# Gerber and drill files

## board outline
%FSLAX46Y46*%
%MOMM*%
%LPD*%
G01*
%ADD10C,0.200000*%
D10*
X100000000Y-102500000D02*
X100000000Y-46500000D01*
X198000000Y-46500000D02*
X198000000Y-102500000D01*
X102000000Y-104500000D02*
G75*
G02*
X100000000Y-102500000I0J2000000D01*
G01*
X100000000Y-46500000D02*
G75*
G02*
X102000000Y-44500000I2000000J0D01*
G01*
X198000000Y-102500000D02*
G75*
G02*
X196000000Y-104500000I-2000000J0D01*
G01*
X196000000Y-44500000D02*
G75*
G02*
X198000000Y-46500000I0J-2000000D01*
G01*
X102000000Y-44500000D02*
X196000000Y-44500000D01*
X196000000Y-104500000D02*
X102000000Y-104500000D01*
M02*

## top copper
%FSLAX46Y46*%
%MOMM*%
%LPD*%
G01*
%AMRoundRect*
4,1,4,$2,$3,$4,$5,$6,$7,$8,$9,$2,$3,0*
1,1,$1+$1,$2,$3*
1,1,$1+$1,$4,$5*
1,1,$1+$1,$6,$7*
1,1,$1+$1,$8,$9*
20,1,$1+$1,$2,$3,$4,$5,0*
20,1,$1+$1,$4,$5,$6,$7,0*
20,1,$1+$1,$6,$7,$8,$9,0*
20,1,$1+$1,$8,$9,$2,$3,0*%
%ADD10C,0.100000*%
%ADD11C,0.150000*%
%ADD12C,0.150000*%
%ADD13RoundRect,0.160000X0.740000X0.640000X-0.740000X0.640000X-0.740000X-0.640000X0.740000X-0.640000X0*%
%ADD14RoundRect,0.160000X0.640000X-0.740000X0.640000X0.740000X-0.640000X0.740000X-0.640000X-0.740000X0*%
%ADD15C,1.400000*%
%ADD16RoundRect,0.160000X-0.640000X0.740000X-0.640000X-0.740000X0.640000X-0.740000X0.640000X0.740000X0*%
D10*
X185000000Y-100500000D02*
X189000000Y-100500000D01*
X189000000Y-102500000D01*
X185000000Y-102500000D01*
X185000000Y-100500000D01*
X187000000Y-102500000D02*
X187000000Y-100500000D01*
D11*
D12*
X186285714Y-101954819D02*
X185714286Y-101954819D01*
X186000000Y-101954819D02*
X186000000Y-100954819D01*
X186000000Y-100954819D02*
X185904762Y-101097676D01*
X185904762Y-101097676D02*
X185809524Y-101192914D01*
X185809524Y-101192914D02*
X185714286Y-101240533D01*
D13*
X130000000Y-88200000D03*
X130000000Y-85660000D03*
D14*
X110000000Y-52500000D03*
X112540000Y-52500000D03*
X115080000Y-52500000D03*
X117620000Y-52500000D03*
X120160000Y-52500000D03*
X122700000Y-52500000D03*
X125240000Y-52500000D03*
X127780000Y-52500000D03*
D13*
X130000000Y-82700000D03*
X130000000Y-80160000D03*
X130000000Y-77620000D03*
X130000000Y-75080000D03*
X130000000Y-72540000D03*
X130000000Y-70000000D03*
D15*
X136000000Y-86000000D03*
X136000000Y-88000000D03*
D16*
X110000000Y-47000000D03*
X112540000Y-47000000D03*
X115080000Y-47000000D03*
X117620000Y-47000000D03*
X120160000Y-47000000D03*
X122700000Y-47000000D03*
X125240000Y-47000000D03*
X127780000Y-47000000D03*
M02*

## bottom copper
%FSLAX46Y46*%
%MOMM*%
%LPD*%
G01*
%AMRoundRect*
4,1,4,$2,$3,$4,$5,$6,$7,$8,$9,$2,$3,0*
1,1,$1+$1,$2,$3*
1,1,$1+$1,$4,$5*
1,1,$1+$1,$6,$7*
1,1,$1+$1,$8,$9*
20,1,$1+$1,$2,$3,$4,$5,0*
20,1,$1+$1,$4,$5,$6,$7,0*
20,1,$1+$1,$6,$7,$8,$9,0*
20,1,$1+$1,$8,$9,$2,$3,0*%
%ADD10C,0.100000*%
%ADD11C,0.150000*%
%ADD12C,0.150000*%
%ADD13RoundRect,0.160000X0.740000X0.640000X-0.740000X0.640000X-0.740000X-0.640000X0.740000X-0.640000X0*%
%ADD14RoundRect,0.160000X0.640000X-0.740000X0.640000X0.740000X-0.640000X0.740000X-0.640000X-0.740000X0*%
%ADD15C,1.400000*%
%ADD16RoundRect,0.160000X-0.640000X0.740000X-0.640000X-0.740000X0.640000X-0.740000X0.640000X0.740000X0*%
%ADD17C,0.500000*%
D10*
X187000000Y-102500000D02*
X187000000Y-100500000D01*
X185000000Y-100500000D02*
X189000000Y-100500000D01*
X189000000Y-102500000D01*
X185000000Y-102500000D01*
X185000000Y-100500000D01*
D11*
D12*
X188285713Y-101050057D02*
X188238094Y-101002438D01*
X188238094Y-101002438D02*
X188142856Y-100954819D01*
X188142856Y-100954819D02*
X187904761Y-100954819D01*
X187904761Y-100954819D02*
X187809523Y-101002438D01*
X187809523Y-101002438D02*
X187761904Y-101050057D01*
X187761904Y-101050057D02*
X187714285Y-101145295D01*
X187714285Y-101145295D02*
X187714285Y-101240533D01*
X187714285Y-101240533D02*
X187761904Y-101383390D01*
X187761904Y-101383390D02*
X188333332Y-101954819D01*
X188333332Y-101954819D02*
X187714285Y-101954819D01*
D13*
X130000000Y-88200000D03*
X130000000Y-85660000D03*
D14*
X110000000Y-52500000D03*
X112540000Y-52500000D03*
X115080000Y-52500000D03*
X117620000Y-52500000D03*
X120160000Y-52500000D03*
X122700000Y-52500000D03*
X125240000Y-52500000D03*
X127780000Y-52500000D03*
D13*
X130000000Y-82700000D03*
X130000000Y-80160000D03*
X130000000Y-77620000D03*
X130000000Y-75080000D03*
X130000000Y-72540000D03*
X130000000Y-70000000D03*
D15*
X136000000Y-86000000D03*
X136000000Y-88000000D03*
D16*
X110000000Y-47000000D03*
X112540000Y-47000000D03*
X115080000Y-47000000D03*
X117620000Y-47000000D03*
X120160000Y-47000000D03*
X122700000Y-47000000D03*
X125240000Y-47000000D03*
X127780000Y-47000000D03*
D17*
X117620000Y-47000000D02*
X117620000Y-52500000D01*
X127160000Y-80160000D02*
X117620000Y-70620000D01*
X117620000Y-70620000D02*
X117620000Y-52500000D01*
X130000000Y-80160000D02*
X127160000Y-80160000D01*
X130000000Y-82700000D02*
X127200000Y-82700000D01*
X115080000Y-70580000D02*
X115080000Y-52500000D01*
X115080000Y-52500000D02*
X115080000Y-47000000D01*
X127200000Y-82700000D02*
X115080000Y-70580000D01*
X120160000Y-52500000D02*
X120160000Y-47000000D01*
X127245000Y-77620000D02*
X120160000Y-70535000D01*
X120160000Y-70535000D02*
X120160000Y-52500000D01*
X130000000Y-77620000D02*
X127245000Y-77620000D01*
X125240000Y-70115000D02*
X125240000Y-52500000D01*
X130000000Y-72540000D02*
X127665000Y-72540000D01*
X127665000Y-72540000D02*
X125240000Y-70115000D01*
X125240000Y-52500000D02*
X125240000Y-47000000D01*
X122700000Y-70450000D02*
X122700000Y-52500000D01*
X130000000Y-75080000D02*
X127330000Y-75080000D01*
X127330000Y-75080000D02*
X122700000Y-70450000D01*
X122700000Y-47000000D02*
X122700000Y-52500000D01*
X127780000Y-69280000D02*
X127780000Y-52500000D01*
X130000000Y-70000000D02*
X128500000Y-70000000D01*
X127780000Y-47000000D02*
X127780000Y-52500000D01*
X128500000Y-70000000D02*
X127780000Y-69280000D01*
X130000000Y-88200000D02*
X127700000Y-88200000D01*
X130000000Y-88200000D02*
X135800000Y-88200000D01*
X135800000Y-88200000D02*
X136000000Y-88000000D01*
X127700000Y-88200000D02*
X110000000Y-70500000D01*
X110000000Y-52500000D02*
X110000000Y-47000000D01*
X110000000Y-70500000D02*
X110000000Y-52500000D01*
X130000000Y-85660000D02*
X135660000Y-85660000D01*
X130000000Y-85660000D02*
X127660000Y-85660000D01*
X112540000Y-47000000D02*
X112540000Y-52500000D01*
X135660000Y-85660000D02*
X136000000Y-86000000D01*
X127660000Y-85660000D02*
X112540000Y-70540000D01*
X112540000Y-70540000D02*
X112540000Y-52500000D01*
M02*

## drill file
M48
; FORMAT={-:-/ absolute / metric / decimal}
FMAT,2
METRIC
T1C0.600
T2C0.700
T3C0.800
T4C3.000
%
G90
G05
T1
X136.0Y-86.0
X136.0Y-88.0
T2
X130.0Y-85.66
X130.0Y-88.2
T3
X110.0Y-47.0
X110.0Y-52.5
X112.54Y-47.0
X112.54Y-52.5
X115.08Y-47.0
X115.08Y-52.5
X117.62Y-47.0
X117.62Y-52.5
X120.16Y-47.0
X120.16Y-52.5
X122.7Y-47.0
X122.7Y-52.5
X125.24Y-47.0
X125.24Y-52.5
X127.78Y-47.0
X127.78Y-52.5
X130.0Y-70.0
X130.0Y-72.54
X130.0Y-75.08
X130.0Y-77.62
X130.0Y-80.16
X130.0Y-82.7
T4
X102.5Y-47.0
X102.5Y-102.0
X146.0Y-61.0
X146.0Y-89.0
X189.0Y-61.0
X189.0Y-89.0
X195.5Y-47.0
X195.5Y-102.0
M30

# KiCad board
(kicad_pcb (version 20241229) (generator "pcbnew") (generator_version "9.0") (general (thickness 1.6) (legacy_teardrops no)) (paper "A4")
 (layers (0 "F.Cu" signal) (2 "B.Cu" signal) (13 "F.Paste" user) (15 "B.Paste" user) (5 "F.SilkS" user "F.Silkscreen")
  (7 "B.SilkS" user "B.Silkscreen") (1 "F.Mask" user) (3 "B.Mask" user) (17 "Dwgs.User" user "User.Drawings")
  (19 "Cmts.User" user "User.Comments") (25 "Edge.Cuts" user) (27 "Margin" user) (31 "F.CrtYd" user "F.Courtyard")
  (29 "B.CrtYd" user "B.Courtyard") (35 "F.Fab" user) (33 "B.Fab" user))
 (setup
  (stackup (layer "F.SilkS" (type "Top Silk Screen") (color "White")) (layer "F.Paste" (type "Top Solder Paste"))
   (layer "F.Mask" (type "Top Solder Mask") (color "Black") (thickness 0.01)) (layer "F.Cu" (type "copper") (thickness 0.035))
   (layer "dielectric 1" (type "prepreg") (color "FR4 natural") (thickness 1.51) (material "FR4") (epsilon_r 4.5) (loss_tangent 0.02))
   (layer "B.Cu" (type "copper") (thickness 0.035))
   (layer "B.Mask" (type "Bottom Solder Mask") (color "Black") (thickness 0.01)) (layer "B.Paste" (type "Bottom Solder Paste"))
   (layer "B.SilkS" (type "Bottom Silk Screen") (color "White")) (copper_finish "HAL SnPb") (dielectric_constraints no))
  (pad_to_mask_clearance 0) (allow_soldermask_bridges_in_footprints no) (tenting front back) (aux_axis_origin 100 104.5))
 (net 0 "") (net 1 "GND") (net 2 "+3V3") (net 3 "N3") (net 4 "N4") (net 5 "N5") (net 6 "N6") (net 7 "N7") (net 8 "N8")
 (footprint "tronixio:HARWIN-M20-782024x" (layer "F.Cu") (at 130 88.2 180)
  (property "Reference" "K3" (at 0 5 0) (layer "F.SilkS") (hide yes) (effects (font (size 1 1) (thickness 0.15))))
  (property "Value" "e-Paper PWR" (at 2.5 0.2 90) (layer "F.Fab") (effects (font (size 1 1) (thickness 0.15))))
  (pad "1" thru_hole roundrect (at 0 0 180) (size 1.8 1.6) (drill 0.7) (layers "*.Cu" "*.Mask") (remove_unused_layers no)
   (roundrect_rratio 0.1) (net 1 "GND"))
  (pad "2" thru_hole roundrect (at 0 2.54 180) (size 1.8 1.6) (drill 0.7) (layers "*.Cu" "*.Mask") (remove_unused_layers no)
   (roundrect_rratio 0.1) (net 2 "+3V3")))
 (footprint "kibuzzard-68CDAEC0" (layer "F.Cu") (at 112.54 57 90)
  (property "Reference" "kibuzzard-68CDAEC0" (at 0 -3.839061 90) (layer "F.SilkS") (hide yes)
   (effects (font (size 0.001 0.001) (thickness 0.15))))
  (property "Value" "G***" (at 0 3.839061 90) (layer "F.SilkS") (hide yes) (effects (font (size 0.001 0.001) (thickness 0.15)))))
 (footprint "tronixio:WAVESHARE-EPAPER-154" (layer "F.Cu") (at 167.5 75)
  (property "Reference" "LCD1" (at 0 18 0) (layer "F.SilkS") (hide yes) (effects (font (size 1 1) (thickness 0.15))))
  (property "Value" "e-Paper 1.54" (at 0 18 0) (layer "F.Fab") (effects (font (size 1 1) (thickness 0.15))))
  (pad "" np_thru_hole circle (at -21.5 -14) (size 3 3) (drill 3) (layers "*.Cu" "*.Mask"))
  (pad "" np_thru_hole circle (at -21.5 14) (size 3 3) (drill 3) (layers "*.Cu" "*.Mask"))
  (pad "" np_thru_hole circle (at 21.5 -14) (size 3 3) (drill 3) (layers "*.Cu" "*.Mask"))
  (pad "" np_thru_hole circle (at 21.5 14) (size 3 3) (drill 3) (layers "*.Cu" "*.Mask")))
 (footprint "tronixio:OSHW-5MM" (layer "F.Cu") (at 167.5 67.5)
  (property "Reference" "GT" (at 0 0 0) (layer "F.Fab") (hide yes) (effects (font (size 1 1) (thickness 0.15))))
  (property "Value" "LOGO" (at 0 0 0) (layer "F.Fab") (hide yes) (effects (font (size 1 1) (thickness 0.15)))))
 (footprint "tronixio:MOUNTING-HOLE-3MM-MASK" (layer "F.Cu") (at 195.5 102)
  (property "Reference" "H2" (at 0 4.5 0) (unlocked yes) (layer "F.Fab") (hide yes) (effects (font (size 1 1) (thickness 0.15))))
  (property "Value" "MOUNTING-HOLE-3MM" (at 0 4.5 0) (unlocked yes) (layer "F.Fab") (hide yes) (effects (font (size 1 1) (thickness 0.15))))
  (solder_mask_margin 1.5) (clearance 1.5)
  (pad "" np_thru_hole circle (at 0 0) (size 3 3) (drill 3) (layers "*.Cu" "*.Mask")))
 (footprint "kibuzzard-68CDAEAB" (layer "F.Cu") (at 126 88.5)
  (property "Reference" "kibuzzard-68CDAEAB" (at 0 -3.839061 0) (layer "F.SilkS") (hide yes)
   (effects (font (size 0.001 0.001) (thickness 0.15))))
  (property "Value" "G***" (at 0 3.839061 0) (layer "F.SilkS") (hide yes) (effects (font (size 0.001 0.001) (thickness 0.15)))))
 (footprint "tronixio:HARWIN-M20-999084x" (layer "F.Cu") (at 110 52.5 90)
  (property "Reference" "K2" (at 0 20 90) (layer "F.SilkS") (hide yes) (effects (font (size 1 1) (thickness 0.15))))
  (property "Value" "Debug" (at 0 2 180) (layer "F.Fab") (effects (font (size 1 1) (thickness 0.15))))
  (pad "1" thru_hole roundrect (at 0 0 90) (size 1.8 1.6) (drill 0.8) (layers "*.Cu" "*.Mask") (remove_unused_layers no)
   (roundrect_rratio 0.1) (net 1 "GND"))
  (pad "2" thru_hole roundrect (at 0 2.54 90) (size 1.8 1.6) (drill 0.8) (layers "*.Cu" "*.Mask") (remove_unused_layers no)
   (roundrect_rratio 0.1) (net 2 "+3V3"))
  (pad "3" thru_hole roundrect (at 0 5.08 90) (size 1.8 1.6) (drill 0.8) (layers "*.Cu" "*.Mask") (remove_unused_layers no)
   (roundrect_rratio 0.1) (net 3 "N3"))
  (pad "4" thru_hole roundrect (at 0 7.62 90) (size 1.8 1.6) (drill 0.8) (layers "*.Cu" "*.Mask") (remove_unused_layers no)
   (roundrect_rratio 0.1) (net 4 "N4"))
  (pad "5" thru_hole roundrect (at 0 10.16 90) (size 1.8 1.6) (drill 0.8) (layers "*.Cu" "*.Mask") (remove_unused_layers no)
   (roundrect_rratio 0.1) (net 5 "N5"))
  (pad "6" thru_hole roundrect (at 0 12.7 90) (size 1.8 1.6) (drill 0.8) (layers "*.Cu" "*.Mask") (remove_unused_layers no)
   (roundrect_rratio 0.1) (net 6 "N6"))
  (pad "7" thru_hole roundrect (at 0 15.24 90) (size 1.8 1.6) (drill 0.8) (layers "*.Cu" "*.Mask") (remove_unused_layers no)
   (roundrect_rratio 0.1) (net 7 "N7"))
  (pad "8" thru_hole roundrect (at 0 17.78 90) (size 1.8 1.6) (drill 0.8) (layers "*.Cu" "*.Mask") (remove_unused_layers no)
   (roundrect_rratio 0.1) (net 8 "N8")))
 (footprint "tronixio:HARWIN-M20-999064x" (layer "F.Cu") (at 130 82.7 180)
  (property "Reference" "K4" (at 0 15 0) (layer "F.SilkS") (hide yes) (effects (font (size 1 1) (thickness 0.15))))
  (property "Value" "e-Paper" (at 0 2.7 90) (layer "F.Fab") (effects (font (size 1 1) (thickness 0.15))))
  (pad "1" thru_hole roundrect (at 0 0 180) (size 1.8 1.6) (drill 0.8) (layers "*.Cu" "*.Mask") (remove_unused_layers no)
   (roundrect_rratio 0.1) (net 3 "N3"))
  (pad "2" thru_hole roundrect (at 0 2.54 180) (size 1.8 1.6) (drill 0.8) (layers "*.Cu" "*.Mask") (remove_unused_layers no)
   (roundrect_rratio 0.1) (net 4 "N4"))
  (pad "3" thru_hole roundrect (at 0 5.08 180) (size 1.8 1.6) (drill 0.8) (layers "*.Cu" "*.Mask") (remove_unused_layers no)
   (roundrect_rratio 0.1) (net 5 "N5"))
  (pad "4" thru_hole roundrect (at 0 7.62 180) (size 1.8 1.6) (drill 0.8) (layers "*.Cu" "*.Mask") (remove_unused_layers no)
   (roundrect_rratio 0.1) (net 6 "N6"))
  (pad "5" thru_hole roundrect (at 0 10.16 180) (size 1.8 1.6) (drill 0.8) (layers "*.Cu" "*.Mask") (remove_unused_layers no)
   (roundrect_rratio 0.1) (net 7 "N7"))
  (pad "6" thru_hole roundrect (at 0 12.7 180) (size 1.8 1.6) (drill 0.8) (layers "*.Cu" "*.Mask") (remove_unused_layers no)
   (roundrect_rratio 0.1) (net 8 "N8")))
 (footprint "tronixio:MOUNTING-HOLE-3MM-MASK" (layer "F.Cu") (at 102.5 47)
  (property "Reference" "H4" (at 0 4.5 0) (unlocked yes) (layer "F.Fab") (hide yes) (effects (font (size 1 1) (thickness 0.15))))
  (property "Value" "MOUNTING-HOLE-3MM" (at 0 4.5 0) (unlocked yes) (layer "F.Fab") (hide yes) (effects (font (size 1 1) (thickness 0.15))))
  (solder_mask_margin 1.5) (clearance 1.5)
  (pad "" np_thru_hole circle (at 0 0) (size 3 3) (drill 3) (layers "*.Cu" "*.Mask")))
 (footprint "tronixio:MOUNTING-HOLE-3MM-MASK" (layer "F.Cu") (at 195.5 47)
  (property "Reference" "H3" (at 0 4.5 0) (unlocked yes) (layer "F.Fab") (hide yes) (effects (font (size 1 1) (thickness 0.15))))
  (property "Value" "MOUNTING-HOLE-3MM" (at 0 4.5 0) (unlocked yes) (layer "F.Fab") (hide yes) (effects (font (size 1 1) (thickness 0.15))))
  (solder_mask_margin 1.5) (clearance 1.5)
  (pad "" np_thru_hole circle (at 0 0) (size 3 3) (drill 3) (layers "*.Cu" "*.Mask")))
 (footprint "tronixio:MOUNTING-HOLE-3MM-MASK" (layer "F.Cu") (at 102.5 102)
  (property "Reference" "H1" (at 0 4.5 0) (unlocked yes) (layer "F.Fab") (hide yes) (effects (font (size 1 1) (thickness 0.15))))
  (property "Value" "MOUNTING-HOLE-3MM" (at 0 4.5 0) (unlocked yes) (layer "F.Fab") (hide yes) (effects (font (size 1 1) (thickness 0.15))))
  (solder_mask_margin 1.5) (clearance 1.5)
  (pad "" np_thru_hole circle (at 0 0) (size 3 3) (drill 3) (layers "*.Cu" "*.Mask")))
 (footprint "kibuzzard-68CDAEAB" (layer "F.Cu") (at 110 56.5 90)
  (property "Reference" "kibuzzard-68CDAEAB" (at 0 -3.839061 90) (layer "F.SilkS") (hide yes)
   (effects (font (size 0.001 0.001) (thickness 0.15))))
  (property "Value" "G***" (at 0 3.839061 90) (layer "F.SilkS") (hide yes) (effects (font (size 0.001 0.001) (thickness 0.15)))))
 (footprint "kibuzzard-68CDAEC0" (layer "F.Cu") (at 125.75 85.66)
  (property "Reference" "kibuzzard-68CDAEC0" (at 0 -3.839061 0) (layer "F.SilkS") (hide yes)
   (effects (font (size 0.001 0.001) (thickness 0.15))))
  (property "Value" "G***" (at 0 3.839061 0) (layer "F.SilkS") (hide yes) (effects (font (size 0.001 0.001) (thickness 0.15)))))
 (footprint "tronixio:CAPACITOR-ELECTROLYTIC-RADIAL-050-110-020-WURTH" (layer "F.Cu") (at 136 87 -90)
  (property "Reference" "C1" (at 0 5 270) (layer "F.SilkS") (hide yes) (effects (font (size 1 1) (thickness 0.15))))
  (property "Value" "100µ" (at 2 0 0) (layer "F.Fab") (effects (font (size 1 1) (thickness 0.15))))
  (pad "1" thru_hole circle (at -1 0 270) (size 1.4 1.4) (drill 0.6) (layers "*.Cu" "*.Mask") (remove_unused_layers no) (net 2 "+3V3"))
  (pad "2" thru_hole circle (at 1 0 270) (size 1.4 1.4) (drill 0.6) (layers "*.Cu" "*.Mask") (remove_unused_layers no) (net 1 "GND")))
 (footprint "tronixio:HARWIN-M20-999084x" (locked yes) (layer "B.Cu") (at 110 47 -90)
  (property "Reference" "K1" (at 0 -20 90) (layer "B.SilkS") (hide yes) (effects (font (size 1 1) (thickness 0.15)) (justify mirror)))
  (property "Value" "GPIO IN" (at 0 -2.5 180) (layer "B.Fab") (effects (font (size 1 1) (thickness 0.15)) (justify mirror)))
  (pad "1" thru_hole roundrect (at 0 0 270) (size 1.8 1.6) (drill 0.8) (layers "*.Cu" "*.Mask") (remove_unused_layers no)
   (roundrect_rratio 0.1) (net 1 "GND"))
  (pad "2" thru_hole roundrect (at 0 -2.54 270) (size 1.8 1.6) (drill 0.8) (layers "*.Cu" "*.Mask") (remove_unused_layers no)
   (roundrect_rratio 0.1) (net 2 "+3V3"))
  (pad "3" thru_hole roundrect (at 0 -5.08 270) (size 1.8 1.6) (drill 0.8) (layers "*.Cu" "*.Mask") (remove_unused_layers no)
   (roundrect_rratio 0.1) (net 3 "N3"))
  (pad "4" thru_hole roundrect (at 0 -7.62 270) (size 1.8 1.6) (drill 0.8) (layers "*.Cu" "*.Mask") (remove_unused_layers no)
   (roundrect_rratio 0.1) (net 4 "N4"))
  (pad "5" thru_hole roundrect (at 0 -10.16 270) (size 1.8 1.6) (drill 0.8) (layers "*.Cu" "*.Mask") (remove_unused_layers no)
   (roundrect_rratio 0.1) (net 5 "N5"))
  (pad "6" thru_hole roundrect (at 0 -12.7 270) (size 1.8 1.6) (drill 0.8) (layers "*.Cu" "*.Mask") (remove_unused_layers no)
   (roundrect_rratio 0.1) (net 6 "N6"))
  (pad "7" thru_hole roundrect (at 0 -15.24 270) (size 1.8 1.6) (drill 0.8) (layers "*.Cu" "*.Mask") (remove_unused_layers no)
   (roundrect_rratio 0.1) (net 7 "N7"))
  (pad "8" thru_hole roundrect (at 0 -17.78 270) (size 1.8 1.6) (drill 0.8) (layers "*.Cu" "*.Mask") (remove_unused_layers no)
   (roundrect_rratio 0.1) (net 8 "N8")))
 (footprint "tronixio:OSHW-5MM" (layer "B.Cu") (at 167.5 67.5 180)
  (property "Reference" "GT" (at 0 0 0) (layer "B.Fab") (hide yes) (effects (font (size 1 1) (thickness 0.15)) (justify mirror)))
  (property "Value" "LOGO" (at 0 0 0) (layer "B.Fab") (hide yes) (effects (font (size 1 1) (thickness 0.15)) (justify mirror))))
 (gr_rect (start 185 100.5) (end 189 102.5) (stroke (width 0.1) (type solid)) (fill no) (layer "F.Cu"))
 (gr_line (start 187 102.5) (end 187 100.5) (stroke (width 0.1) (type solid)) (layer "F.Cu"))
 (gr_line (start 187 102.5) (end 187 100.5) (stroke (width 0.1) (type solid)) (layer "B.Cu"))
 (gr_rect (start 185 100.5) (end 189 102.5) (stroke (width 0.1) (type solid)) (fill no) (layer "B.Cu"))
 (gr_line (start 100 102.5) (end 100 46.5) (stroke (width 0.2) (type default)) (layer "Edge.Cuts"))
 (gr_line (start 198 46.5) (end 198 102.5) (stroke (width 0.2) (type default)) (layer "Edge.Cuts"))
 (gr_arc (start 102 104.5) (mid 100.585786 103.914214) (end 100 102.5) (stroke (width 0.2) (type default)) (layer "Edge.Cuts"))
 (gr_arc (start 100 46.5) (mid 100.585786 45.085786) (end 102 44.5) (stroke (width 0.2) (type default)) (layer "Edge.Cuts"))
 (gr_arc (start 198 102.5) (mid 197.414214 103.914214) (end 196 104.5) (stroke (width 0.2) (type default)) (layer "Edge.Cuts"))
 (gr_arc (start 196 44.5) (mid 197.414214 45.085786) (end 198 46.5) (stroke (width 0.2) (type default)) (layer "Edge.Cuts"))
 (gr_line (start 102 44.5) (end 196 44.5) (stroke (width 0.2) (type default)) (layer "Edge.Cuts"))
 (gr_line (start 196 104.5) (end 102 104.5) (stroke (width 0.2) (type default)) (layer "Edge.Cuts"))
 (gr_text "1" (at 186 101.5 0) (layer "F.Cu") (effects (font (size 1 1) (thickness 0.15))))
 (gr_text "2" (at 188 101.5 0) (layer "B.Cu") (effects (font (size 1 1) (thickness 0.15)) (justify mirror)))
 (segment (start 117.62 47) (end 117.62 52.5) (width 0.5) (layer "B.Cu") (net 4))
 (segment (start 127.16 80.16) (end 117.62 70.62) (width 0.5) (layer "B.Cu") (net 4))
 (segment (start 117.62 70.62) (end 117.62 52.5) (width 0.5) (layer "B.Cu") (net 4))
 (segment (start 130 80.16) (end 127.16 80.16) (width 0.5) (layer "B.Cu") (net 4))
 (segment (start 130 82.7) (end 127.2 82.7) (width 0.5) (layer "B.Cu") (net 3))
 (segment (start 115.08 70.58) (end 115.08 52.5) (width 0.5) (layer "B.Cu") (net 3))
 (segment (start 115.08 52.5) (end 115.08 47) (width 0.5) (layer "B.Cu") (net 3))
 (segment (start 127.2 82.7) (end 115.08 70.58) (width 0.5) (layer "B.Cu") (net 3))
 (segment (start 120.16 52.5) (end 120.16 47) (width 0.5) (layer "B.Cu") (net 5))
 (segment (start 127.245 77.62) (end 120.16 70.535) (width 0.5) (layer "B.Cu") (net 5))
 (segment (start 120.16 70.535) (end 120.16 52.5) (width 0.5) (layer "B.Cu") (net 5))
 (segment (start 130 77.62) (end 127.245 77.62) (width 0.5) (layer "B.Cu") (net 5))
 (segment (start 125.24 70.115) (end 125.24 52.5) (width 0.5) (layer "B.Cu") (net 7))
 (segment (start 130 72.54) (end 127.665 72.54) (width 0.5) (layer "B.Cu") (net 7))
 (segment (start 127.665 72.54) (end 125.24 70.115) (width 0.5) (layer "B.Cu") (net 7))
 (segment (start 125.24 52.5) (end 125.24 47) (width 0.5) (layer "B.Cu") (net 7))
 (segment (start 122.7 70.45) (end 122.7 52.5) (width 0.5) (layer "B.Cu") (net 6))
 (segment (start 130 75.08) (end 127.33 75.08) (width 0.5) (layer "B.Cu") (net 6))
 (segment (start 127.33 75.08) (end 122.7 70.45) (width 0.5) (layer "B.Cu") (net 6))
 (segment (start 122.7 47) (end 122.7 52.5) (width 0.5) (layer "B.Cu") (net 6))
 (segment (start 127.78 69.28) (end 127.78 52.5) (width 0.5) (layer "B.Cu") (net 8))
 (segment (start 130 70) (end 128.5 70) (width 0.5) (layer "B.Cu") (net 8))
 (segment (start 127.78 47) (end 127.78 52.5) (width 0.5) (layer "B.Cu") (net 8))
 (segment (start 128.5 70) (end 127.78 69.28) (width 0.5) (layer "B.Cu") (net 8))
 (segment (start 130 88.2) (end 127.7 88.2) (width 0.5) (layer "B.Cu") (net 1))
 (segment (start 130 88.2) (end 135.8 88.2) (width 0.5) (layer "B.Cu") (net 1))
 (segment (start 135.8 88.2) (end 136 88) (width 0.5) (layer "B.Cu") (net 1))
 (segment (start 127.7 88.2) (end 110 70.5) (width 0.5) (layer "B.Cu") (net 1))
 (segment (start 110 52.5) (end 110 47) (width 0.5) (layer "B.Cu") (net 1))
 (segment (start 110 70.5) (end 110 52.5) (width 0.5) (layer "B.Cu") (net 1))
 (segment (start 130 85.66) (end 135.66 85.66) (width 0.5) (layer "B.Cu") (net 2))
 (segment (start 130 85.66) (end 127.66 85.66) (width 0.5) (layer "B.Cu") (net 2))
 (segment (start 112.54 47) (end 112.54 52.5) (width 0.5) (layer "B.Cu") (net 2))
 (segment (start 135.66 85.66) (end 136 86) (width 0.5) (layer "B.Cu") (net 2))
 (segment (start 127.66 85.66) (end 112.54 70.54) (width 0.5) (layer "B.Cu") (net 2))
 (segment (start 112.54 70.54) (end 112.54 52.5) (width 0.5) (layer "B.Cu") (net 2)))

